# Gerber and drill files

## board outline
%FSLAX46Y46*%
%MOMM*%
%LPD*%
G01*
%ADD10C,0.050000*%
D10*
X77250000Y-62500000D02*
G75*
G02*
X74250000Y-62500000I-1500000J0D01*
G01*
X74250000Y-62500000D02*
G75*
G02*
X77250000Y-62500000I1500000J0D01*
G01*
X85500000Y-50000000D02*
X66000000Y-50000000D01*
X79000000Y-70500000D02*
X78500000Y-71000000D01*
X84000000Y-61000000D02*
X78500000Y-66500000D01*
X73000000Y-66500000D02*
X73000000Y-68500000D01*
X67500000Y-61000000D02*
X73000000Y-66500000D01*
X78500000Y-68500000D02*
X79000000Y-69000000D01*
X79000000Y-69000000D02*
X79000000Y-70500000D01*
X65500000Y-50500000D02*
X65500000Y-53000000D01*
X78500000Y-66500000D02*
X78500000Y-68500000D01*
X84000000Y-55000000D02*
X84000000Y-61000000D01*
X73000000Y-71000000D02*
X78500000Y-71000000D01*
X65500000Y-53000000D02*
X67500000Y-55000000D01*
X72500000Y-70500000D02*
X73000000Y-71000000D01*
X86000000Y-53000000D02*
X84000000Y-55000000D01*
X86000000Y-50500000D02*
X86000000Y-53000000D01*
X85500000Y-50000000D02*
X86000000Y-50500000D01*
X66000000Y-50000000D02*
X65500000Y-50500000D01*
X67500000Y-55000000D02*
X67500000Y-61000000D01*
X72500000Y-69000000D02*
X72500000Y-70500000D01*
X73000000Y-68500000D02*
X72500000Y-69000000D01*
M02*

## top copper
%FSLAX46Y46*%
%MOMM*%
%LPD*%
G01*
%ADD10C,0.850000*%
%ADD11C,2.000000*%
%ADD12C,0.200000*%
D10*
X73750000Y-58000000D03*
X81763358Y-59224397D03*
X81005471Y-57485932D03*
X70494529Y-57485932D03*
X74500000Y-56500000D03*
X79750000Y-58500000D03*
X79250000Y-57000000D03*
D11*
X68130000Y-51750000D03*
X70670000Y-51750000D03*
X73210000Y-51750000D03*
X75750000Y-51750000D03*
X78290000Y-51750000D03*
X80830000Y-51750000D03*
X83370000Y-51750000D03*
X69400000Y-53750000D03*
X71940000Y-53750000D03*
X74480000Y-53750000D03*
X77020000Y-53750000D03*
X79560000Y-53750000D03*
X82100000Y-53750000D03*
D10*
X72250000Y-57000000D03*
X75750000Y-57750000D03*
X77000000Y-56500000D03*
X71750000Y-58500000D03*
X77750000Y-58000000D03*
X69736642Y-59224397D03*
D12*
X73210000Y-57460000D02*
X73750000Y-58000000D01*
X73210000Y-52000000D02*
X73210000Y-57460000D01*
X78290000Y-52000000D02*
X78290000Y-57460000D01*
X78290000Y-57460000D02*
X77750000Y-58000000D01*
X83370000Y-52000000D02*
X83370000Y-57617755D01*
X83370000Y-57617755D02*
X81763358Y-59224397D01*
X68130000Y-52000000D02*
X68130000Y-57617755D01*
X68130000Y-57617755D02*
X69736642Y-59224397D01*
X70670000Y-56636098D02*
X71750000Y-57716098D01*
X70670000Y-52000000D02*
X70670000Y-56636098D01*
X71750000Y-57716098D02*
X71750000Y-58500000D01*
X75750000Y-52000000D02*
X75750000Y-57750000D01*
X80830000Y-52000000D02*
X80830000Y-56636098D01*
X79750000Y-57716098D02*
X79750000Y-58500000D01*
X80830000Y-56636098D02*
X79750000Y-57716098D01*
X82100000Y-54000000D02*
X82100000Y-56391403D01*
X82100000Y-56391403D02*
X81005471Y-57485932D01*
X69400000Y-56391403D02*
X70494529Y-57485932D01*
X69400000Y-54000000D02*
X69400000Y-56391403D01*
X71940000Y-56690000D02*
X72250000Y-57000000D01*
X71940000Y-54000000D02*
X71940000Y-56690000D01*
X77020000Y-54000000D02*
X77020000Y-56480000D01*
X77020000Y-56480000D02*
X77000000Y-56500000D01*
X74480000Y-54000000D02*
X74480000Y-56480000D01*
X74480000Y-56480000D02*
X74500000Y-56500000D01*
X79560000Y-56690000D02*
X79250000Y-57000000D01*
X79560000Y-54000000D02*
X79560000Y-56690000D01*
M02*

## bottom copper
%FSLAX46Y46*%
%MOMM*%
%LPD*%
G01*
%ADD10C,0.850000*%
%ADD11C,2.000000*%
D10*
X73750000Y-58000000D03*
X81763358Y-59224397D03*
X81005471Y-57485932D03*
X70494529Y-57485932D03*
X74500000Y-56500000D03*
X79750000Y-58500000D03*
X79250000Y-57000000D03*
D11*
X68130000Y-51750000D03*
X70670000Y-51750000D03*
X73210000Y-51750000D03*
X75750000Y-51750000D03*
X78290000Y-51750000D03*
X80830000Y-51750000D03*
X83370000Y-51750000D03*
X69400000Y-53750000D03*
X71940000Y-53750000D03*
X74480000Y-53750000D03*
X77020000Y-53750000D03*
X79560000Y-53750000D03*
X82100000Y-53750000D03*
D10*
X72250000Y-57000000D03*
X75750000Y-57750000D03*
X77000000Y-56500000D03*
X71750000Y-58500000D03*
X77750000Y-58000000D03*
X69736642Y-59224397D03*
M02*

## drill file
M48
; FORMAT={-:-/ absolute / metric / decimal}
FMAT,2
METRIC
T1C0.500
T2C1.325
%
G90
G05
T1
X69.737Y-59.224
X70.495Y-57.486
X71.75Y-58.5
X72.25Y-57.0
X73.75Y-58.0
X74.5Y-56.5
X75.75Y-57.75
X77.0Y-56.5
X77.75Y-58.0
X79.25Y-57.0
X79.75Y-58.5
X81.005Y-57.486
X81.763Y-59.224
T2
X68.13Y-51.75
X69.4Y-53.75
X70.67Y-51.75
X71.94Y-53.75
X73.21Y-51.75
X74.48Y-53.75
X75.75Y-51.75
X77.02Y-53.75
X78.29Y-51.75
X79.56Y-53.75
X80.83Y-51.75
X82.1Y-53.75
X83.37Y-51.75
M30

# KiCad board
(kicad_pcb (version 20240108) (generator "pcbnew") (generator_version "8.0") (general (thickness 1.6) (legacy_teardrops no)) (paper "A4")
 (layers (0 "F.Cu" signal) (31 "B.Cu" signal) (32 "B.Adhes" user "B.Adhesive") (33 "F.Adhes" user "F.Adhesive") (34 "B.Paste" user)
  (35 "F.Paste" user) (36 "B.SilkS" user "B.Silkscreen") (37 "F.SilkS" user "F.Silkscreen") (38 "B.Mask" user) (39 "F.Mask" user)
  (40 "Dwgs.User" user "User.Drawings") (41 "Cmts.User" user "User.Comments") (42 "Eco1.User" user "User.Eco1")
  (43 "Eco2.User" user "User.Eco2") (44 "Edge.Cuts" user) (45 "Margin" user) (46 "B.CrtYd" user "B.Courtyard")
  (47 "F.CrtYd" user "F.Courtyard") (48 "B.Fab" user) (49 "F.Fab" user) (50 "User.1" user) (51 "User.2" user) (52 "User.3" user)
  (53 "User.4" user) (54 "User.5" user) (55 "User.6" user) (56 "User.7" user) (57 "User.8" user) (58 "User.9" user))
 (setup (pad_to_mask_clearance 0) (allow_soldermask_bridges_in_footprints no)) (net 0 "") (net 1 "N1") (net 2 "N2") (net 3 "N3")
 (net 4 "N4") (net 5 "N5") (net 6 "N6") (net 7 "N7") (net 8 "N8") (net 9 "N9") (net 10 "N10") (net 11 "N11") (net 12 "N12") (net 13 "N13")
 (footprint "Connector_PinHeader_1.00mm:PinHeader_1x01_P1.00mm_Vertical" (layer "F.Cu") (at 73.75 58)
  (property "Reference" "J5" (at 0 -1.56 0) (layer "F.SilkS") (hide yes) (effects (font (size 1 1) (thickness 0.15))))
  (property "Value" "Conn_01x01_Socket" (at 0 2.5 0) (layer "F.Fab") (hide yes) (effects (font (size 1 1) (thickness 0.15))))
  (pad "1" thru_hole circle (at 0 0) (size 0.85 0.85) (drill 0.5) (layers "*.Cu" "*.Mask") (remove_unused_layers no) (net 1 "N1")))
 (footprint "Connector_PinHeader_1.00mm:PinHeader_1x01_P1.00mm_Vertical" (layer "F.Cu") (at 81.763358 59.224397)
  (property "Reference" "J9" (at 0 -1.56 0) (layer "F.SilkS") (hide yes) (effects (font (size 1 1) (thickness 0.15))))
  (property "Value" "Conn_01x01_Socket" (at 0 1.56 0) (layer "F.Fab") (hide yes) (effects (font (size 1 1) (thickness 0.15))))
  (pad "1" thru_hole circle (at 0 0) (size 0.85 0.85) (drill 0.5) (layers "*.Cu" "*.Mask") (remove_unused_layers no) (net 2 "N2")))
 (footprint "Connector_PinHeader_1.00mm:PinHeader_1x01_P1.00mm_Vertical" (layer "F.Cu") (at 81.005471 57.485932)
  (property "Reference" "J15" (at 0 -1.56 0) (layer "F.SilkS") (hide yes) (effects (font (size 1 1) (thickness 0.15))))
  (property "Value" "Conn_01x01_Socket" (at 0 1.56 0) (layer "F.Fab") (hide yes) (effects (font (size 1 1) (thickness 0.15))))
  (pad "1" thru_hole circle (at 0 0) (size 0.85 0.85) (drill 0.5) (layers "*.Cu" "*.Mask") (remove_unused_layers no) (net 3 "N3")))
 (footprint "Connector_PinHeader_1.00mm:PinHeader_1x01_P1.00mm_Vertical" (layer "F.Cu") (at 70.494529 57.485932)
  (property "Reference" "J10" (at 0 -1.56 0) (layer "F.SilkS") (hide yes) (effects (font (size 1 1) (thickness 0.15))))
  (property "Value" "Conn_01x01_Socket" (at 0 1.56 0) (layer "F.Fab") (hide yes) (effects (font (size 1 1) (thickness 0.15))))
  (pad "1" thru_hole circle (at 0 0) (size 0.85 0.85) (drill 0.5) (layers "*.Cu" "*.Mask") (remove_unused_layers no) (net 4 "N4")))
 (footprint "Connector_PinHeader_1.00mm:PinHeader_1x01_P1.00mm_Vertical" (layer "F.Cu") (at 74.5 56.5)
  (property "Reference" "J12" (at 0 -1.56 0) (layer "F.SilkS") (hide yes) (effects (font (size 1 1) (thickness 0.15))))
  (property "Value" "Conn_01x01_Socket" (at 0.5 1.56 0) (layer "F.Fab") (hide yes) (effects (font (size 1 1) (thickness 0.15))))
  (pad "1" thru_hole circle (at 0 0) (size 0.85 0.85) (drill 0.5) (layers "*.Cu" "*.Mask") (remove_unused_layers no) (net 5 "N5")))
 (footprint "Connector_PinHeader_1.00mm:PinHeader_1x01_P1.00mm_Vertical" (layer "F.Cu") (at 79.75 58.5)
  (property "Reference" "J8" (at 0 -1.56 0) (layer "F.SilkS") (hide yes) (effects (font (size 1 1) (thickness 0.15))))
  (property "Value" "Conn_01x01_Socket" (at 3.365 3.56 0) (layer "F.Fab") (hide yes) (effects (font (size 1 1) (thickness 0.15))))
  (pad "1" thru_hole circle (at 0 0) (size 0.85 0.85) (drill 0.5) (layers "*.Cu" "*.Mask") (remove_unused_layers no) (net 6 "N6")))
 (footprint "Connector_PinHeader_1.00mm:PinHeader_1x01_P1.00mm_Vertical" (layer "F.Cu") (at 79.25 57)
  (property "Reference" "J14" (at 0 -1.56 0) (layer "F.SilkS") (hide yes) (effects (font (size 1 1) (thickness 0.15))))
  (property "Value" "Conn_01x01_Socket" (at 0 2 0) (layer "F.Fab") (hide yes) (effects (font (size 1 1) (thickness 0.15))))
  (pad "1" thru_hole circle (at 0 0) (size 0.85 0.85) (drill 0.5) (layers "*.Cu" "*.Mask") (remove_unused_layers no) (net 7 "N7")))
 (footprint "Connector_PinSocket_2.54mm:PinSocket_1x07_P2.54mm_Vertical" (layer "F.Cu") (at 68.13 51.75 90)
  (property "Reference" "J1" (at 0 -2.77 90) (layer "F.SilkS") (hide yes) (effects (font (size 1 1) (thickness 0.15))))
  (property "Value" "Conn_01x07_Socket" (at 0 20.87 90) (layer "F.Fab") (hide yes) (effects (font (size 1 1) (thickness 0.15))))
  (pad "1" thru_hole circle (at 0 0 90) (size 2 2) (drill 1.325) (layers "*.Cu" "*.Mask") (remove_unused_layers no) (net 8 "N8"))
  (pad "2" thru_hole circle (at 0 2.54 90) (size 2 2) (drill 1.325) (layers "*.Cu" "*.Mask") (remove_unused_layers no) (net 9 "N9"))
  (pad "3" thru_hole circle (at 0 5.08 90) (size 2 2) (drill 1.325) (layers "*.Cu" "*.Mask") (remove_unused_layers no) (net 1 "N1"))
  (pad "4" thru_hole circle (at 0 7.62 90) (size 2 2) (drill 1.325) (layers "*.Cu" "*.Mask") (remove_unused_layers no) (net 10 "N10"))
  (pad "5" thru_hole circle (at 0 10.16 90) (size 2 2) (drill 1.325) (layers "*.Cu" "*.Mask") (remove_unused_layers no) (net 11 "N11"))
  (pad "6" thru_hole circle (at 0 12.7 90) (size 2 2) (drill 1.325) (layers "*.Cu" "*.Mask") (remove_unused_layers no) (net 6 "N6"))
  (pad "7" thru_hole circle (at 0 15.24 90) (size 2 2) (drill 1.325) (layers "*.Cu" "*.Mask") (remove_unused_layers no) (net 2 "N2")))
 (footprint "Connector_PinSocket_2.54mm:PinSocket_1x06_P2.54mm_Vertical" (layer "F.Cu") (at 69.4 53.75 90)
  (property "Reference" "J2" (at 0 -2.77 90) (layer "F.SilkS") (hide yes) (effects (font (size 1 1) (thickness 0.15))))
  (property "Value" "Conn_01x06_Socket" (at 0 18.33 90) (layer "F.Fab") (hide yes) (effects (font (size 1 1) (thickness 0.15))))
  (pad "1" thru_hole circle (at 0 0 90) (size 2 2) (drill 1.325) (layers "*.Cu" "*.Mask") (remove_unused_layers no) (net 4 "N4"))
  (pad "2" thru_hole circle (at 0 2.54 90) (size 2 2) (drill 1.325) (layers "*.Cu" "*.Mask") (remove_unused_layers no) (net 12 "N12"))
  (pad "3" thru_hole circle (at 0 5.08 90) (size 2 2) (drill 1.325) (layers "*.Cu" "*.Mask") (remove_unused_layers no) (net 5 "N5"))
  (pad "4" thru_hole circle (at 0 7.62 90) (size 2 2) (drill 1.325) (layers "*.Cu" "*.Mask") (remove_unused_layers no) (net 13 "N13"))
  (pad "5" thru_hole circle (at 0 10.16 90) (size 2 2) (drill 1.325) (layers "*.Cu" "*.Mask") (remove_unused_layers no) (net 7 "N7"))
  (pad "6" thru_hole circle (at 0 12.7 90) (size 2 2) (drill 1.325) (layers "*.Cu" "*.Mask") (remove_unused_layers no) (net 3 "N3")))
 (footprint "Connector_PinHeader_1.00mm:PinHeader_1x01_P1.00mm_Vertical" (layer "F.Cu") (at 72.25 57)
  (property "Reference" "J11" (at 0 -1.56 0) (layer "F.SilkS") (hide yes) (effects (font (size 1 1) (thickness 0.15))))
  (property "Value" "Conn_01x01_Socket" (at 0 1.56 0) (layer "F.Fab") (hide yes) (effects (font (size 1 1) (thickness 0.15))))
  (pad "1" thru_hole circle (at 0 0) (size 0.85 0.85) (drill 0.5) (layers "*.Cu" "*.Mask") (remove_unused_layers no) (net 12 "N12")))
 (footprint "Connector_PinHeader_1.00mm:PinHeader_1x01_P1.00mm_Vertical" (layer "F.Cu") (at 75.75 57.75)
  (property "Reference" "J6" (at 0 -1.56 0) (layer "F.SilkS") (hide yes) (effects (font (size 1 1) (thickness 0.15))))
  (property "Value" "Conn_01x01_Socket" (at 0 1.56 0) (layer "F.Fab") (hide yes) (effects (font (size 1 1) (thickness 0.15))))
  (pad "1" thru_hole circle (at 0 0) (size 0.85 0.85) (drill 0.5) (layers "*.Cu" "*.Mask") (remove_unused_layers no) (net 10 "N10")))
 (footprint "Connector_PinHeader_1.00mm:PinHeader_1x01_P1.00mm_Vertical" (layer "F.Cu") (at 77 56.5)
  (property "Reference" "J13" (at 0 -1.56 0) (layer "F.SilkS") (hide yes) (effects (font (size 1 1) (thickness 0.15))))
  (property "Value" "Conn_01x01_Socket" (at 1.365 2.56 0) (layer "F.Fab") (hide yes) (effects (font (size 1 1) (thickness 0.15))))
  (pad "1" thru_hole circle (at 0 0) (size 0.85 0.85) (drill 0.5) (layers "*.Cu" "*.Mask") (remove_unused_layers no) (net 13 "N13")))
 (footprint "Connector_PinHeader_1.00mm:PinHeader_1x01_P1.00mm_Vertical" (layer "F.Cu") (at 71.75 58.5)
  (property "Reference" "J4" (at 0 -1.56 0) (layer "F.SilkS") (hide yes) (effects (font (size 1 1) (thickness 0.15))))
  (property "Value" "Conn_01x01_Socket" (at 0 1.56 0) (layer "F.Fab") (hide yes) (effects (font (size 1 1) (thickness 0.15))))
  (pad "1" thru_hole circle (at 0 0) (size 0.85 0.85) (drill 0.5) (layers "*.Cu" "*.Mask") (remove_unused_layers no) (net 9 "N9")))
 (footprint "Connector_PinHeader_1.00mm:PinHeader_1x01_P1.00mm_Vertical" (layer "F.Cu") (at 77.75 58)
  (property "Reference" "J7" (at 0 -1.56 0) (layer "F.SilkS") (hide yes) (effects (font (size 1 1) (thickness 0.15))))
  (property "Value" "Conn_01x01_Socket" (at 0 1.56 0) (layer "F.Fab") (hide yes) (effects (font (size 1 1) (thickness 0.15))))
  (pad "1" thru_hole circle (at 0 0) (size 0.85 0.85) (drill 0.5) (layers "*.Cu" "*.Mask") (remove_unused_layers no) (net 11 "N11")))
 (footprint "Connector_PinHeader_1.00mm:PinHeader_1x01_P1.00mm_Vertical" (layer "F.Cu") (at 69.736642 59.224397)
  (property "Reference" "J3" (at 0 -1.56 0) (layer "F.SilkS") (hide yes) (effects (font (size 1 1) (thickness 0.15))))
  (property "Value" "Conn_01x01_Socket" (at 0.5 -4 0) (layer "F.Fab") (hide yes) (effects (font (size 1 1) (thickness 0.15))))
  (pad "1" thru_hole circle (at 0 0) (size 0.85 0.85) (drill 0.5) (layers "*.Cu" "*.Mask") (remove_unused_layers no) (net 8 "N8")))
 (gr_circle (center 75.75 62.5) (end 75.75 61) (stroke (width 0.05) (type default)) (fill none) (layer "Edge.Cuts"))
 (gr_line (start 85.5 50) (end 66 50) (stroke (width 0.05) (type default)) (layer "Edge.Cuts"))
 (gr_line (start 79 70.5) (end 78.5 71) (stroke (width 0.05) (type default)) (layer "Edge.Cuts"))
 (gr_line (start 84 61) (end 78.5 66.5) (stroke (width 0.05) (type default)) (layer "Edge.Cuts"))
 (gr_line (start 73 66.5) (end 73 68.5) (stroke (width 0.05) (type default)) (layer "Edge.Cuts"))
 (gr_line (start 67.5 61) (end 73 66.5) (stroke (width 0.05) (type default)) (layer "Edge.Cuts"))
 (gr_line (start 78.5 68.5) (end 79 69) (stroke (width 0.05) (type default)) (layer "Edge.Cuts"))
 (gr_line (start 79 69) (end 79 70.5) (stroke (width 0.05) (type default)) (layer "Edge.Cuts"))
 (gr_line (start 65.5 50.5) (end 65.5 53) (stroke (width 0.05) (type default)) (layer "Edge.Cuts"))
 (gr_line (start 78.5 66.5) (end 78.5 68.5) (stroke (width 0.05) (type default)) (layer "Edge.Cuts"))
 (gr_line (start 84 55) (end 84 61) (stroke (width 0.05) (type default)) (layer "Edge.Cuts"))
 (gr_line (start 73 71) (end 78.5 71) (stroke (width 0.05) (type default)) (layer "Edge.Cuts"))
 (gr_line (start 65.5 53) (end 67.5 55) (stroke (width 0.05) (type default)) (layer "Edge.Cuts"))
 (gr_line (start 72.5 70.5) (end 73 71) (stroke (width 0.05) (type default)) (layer "Edge.Cuts"))
 (gr_line (start 86 53) (end 84 55) (stroke (width 0.05) (type default)) (layer "Edge.Cuts"))
 (gr_line (start 86 50.5) (end 86 53) (stroke (width 0.05) (type default)) (layer "Edge.Cuts"))
 (gr_line (start 85.5 50) (end 86 50.5) (stroke (width 0.05) (type default)) (layer "Edge.Cuts"))
 (gr_line (start 66 50) (end 65.5 50.5) (stroke (width 0.05) (type default)) (layer "Edge.Cuts"))
 (gr_line (start 67.5 55) (end 67.5 61) (stroke (width 0.05) (type default)) (layer "Edge.Cuts"))
 (gr_line (start 72.5 69) (end 72.5 70.5) (stroke (width 0.05) (type default)) (layer "Edge.Cuts"))
 (gr_line (start 73 68.5) (end 72.5 69) (stroke (width 0.05) (type default)) (layer "Edge.Cuts"))
 (segment (start 73.21 57.46) (end 73.75 58) (width 0.2) (layer "F.Cu") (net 1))
 (segment (start 73.21 52) (end 73.21 57.46) (width 0.2) (layer "F.Cu") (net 1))
 (segment (start 78.29 52) (end 78.29 57.46) (width 0.2) (layer "F.Cu") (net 11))
 (segment (start 78.29 57.46) (end 77.75 58) (width 0.2) (layer "F.Cu") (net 11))
 (segment (start 83.37 52) (end 83.37 57.617755) (width 0.2) (layer "F.Cu") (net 2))
 (segment (start 83.37 57.617755) (end 81.763358 59.224397) (width 0.2) (layer "F.Cu") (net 2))
 (segment (start 68.13 52) (end 68.13 57.617755) (width 0.2) (layer "F.Cu") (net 8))
 (segment (start 68.13 57.617755) (end 69.736642 59.224397) (width 0.2) (layer "F.Cu") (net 8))
 (segment (start 70.67 56.636098) (end 71.75 57.716098) (width 0.2) (layer "F.Cu") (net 9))
 (segment (start 70.67 52) (end 70.67 56.636098) (width 0.2) (layer "F.Cu") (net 9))
 (segment (start 71.75 57.716098) (end 71.75 58.5) (width 0.2) (layer "F.Cu") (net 9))
 (segment (start 75.75 52) (end 75.75 57.75) (width 0.2) (layer "F.Cu") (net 10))
 (segment (start 80.83 52) (end 80.83 56.636098) (width 0.2) (layer "F.Cu") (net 6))
 (segment (start 79.75 57.716098) (end 79.75 58.5) (width 0.2) (layer "F.Cu") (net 6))
 (segment (start 80.83 56.636098) (end 79.75 57.716098) (width 0.2) (layer "F.Cu") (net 6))
 (segment (start 82.1 54) (end 82.1 56.391403) (width 0.2) (layer "F.Cu") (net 3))
 (segment (start 82.1 56.391403) (end 81.005471 57.485932) (width 0.2) (layer "F.Cu") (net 3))
 (segment (start 69.4 56.391403) (end 70.494529 57.485932) (width 0.2) (layer "F.Cu") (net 4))
 (segment (start 69.4 54) (end 69.4 56.391403) (width 0.2) (layer "F.Cu") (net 4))
 (segment (start 71.94 56.69) (end 72.25 57) (width 0.2) (layer "F.Cu") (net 12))
 (segment (start 71.94 54) (end 71.94 56.69) (width 0.2) (layer "F.Cu") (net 12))
 (segment (start 77.02 54) (end 77.02 56.48) (width 0.2) (layer "F.Cu") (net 13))
 (segment (start 77.02 56.48) (end 77 56.5) (width 0.2) (layer "F.Cu") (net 13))
 (segment (start 74.48 54) (end 74.48 56.48) (width 0.2) (layer "F.Cu") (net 5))
 (segment (start 74.48 56.48) (end 74.5 56.5) (width 0.2) (layer "F.Cu") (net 5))
 (segment (start 79.56 56.69) (end 79.25 57) (width 0.2) (layer "F.Cu") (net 7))
 (segment (start 79.56 54) (end 79.56 56.69) (width 0.2) (layer "F.Cu") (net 7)))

